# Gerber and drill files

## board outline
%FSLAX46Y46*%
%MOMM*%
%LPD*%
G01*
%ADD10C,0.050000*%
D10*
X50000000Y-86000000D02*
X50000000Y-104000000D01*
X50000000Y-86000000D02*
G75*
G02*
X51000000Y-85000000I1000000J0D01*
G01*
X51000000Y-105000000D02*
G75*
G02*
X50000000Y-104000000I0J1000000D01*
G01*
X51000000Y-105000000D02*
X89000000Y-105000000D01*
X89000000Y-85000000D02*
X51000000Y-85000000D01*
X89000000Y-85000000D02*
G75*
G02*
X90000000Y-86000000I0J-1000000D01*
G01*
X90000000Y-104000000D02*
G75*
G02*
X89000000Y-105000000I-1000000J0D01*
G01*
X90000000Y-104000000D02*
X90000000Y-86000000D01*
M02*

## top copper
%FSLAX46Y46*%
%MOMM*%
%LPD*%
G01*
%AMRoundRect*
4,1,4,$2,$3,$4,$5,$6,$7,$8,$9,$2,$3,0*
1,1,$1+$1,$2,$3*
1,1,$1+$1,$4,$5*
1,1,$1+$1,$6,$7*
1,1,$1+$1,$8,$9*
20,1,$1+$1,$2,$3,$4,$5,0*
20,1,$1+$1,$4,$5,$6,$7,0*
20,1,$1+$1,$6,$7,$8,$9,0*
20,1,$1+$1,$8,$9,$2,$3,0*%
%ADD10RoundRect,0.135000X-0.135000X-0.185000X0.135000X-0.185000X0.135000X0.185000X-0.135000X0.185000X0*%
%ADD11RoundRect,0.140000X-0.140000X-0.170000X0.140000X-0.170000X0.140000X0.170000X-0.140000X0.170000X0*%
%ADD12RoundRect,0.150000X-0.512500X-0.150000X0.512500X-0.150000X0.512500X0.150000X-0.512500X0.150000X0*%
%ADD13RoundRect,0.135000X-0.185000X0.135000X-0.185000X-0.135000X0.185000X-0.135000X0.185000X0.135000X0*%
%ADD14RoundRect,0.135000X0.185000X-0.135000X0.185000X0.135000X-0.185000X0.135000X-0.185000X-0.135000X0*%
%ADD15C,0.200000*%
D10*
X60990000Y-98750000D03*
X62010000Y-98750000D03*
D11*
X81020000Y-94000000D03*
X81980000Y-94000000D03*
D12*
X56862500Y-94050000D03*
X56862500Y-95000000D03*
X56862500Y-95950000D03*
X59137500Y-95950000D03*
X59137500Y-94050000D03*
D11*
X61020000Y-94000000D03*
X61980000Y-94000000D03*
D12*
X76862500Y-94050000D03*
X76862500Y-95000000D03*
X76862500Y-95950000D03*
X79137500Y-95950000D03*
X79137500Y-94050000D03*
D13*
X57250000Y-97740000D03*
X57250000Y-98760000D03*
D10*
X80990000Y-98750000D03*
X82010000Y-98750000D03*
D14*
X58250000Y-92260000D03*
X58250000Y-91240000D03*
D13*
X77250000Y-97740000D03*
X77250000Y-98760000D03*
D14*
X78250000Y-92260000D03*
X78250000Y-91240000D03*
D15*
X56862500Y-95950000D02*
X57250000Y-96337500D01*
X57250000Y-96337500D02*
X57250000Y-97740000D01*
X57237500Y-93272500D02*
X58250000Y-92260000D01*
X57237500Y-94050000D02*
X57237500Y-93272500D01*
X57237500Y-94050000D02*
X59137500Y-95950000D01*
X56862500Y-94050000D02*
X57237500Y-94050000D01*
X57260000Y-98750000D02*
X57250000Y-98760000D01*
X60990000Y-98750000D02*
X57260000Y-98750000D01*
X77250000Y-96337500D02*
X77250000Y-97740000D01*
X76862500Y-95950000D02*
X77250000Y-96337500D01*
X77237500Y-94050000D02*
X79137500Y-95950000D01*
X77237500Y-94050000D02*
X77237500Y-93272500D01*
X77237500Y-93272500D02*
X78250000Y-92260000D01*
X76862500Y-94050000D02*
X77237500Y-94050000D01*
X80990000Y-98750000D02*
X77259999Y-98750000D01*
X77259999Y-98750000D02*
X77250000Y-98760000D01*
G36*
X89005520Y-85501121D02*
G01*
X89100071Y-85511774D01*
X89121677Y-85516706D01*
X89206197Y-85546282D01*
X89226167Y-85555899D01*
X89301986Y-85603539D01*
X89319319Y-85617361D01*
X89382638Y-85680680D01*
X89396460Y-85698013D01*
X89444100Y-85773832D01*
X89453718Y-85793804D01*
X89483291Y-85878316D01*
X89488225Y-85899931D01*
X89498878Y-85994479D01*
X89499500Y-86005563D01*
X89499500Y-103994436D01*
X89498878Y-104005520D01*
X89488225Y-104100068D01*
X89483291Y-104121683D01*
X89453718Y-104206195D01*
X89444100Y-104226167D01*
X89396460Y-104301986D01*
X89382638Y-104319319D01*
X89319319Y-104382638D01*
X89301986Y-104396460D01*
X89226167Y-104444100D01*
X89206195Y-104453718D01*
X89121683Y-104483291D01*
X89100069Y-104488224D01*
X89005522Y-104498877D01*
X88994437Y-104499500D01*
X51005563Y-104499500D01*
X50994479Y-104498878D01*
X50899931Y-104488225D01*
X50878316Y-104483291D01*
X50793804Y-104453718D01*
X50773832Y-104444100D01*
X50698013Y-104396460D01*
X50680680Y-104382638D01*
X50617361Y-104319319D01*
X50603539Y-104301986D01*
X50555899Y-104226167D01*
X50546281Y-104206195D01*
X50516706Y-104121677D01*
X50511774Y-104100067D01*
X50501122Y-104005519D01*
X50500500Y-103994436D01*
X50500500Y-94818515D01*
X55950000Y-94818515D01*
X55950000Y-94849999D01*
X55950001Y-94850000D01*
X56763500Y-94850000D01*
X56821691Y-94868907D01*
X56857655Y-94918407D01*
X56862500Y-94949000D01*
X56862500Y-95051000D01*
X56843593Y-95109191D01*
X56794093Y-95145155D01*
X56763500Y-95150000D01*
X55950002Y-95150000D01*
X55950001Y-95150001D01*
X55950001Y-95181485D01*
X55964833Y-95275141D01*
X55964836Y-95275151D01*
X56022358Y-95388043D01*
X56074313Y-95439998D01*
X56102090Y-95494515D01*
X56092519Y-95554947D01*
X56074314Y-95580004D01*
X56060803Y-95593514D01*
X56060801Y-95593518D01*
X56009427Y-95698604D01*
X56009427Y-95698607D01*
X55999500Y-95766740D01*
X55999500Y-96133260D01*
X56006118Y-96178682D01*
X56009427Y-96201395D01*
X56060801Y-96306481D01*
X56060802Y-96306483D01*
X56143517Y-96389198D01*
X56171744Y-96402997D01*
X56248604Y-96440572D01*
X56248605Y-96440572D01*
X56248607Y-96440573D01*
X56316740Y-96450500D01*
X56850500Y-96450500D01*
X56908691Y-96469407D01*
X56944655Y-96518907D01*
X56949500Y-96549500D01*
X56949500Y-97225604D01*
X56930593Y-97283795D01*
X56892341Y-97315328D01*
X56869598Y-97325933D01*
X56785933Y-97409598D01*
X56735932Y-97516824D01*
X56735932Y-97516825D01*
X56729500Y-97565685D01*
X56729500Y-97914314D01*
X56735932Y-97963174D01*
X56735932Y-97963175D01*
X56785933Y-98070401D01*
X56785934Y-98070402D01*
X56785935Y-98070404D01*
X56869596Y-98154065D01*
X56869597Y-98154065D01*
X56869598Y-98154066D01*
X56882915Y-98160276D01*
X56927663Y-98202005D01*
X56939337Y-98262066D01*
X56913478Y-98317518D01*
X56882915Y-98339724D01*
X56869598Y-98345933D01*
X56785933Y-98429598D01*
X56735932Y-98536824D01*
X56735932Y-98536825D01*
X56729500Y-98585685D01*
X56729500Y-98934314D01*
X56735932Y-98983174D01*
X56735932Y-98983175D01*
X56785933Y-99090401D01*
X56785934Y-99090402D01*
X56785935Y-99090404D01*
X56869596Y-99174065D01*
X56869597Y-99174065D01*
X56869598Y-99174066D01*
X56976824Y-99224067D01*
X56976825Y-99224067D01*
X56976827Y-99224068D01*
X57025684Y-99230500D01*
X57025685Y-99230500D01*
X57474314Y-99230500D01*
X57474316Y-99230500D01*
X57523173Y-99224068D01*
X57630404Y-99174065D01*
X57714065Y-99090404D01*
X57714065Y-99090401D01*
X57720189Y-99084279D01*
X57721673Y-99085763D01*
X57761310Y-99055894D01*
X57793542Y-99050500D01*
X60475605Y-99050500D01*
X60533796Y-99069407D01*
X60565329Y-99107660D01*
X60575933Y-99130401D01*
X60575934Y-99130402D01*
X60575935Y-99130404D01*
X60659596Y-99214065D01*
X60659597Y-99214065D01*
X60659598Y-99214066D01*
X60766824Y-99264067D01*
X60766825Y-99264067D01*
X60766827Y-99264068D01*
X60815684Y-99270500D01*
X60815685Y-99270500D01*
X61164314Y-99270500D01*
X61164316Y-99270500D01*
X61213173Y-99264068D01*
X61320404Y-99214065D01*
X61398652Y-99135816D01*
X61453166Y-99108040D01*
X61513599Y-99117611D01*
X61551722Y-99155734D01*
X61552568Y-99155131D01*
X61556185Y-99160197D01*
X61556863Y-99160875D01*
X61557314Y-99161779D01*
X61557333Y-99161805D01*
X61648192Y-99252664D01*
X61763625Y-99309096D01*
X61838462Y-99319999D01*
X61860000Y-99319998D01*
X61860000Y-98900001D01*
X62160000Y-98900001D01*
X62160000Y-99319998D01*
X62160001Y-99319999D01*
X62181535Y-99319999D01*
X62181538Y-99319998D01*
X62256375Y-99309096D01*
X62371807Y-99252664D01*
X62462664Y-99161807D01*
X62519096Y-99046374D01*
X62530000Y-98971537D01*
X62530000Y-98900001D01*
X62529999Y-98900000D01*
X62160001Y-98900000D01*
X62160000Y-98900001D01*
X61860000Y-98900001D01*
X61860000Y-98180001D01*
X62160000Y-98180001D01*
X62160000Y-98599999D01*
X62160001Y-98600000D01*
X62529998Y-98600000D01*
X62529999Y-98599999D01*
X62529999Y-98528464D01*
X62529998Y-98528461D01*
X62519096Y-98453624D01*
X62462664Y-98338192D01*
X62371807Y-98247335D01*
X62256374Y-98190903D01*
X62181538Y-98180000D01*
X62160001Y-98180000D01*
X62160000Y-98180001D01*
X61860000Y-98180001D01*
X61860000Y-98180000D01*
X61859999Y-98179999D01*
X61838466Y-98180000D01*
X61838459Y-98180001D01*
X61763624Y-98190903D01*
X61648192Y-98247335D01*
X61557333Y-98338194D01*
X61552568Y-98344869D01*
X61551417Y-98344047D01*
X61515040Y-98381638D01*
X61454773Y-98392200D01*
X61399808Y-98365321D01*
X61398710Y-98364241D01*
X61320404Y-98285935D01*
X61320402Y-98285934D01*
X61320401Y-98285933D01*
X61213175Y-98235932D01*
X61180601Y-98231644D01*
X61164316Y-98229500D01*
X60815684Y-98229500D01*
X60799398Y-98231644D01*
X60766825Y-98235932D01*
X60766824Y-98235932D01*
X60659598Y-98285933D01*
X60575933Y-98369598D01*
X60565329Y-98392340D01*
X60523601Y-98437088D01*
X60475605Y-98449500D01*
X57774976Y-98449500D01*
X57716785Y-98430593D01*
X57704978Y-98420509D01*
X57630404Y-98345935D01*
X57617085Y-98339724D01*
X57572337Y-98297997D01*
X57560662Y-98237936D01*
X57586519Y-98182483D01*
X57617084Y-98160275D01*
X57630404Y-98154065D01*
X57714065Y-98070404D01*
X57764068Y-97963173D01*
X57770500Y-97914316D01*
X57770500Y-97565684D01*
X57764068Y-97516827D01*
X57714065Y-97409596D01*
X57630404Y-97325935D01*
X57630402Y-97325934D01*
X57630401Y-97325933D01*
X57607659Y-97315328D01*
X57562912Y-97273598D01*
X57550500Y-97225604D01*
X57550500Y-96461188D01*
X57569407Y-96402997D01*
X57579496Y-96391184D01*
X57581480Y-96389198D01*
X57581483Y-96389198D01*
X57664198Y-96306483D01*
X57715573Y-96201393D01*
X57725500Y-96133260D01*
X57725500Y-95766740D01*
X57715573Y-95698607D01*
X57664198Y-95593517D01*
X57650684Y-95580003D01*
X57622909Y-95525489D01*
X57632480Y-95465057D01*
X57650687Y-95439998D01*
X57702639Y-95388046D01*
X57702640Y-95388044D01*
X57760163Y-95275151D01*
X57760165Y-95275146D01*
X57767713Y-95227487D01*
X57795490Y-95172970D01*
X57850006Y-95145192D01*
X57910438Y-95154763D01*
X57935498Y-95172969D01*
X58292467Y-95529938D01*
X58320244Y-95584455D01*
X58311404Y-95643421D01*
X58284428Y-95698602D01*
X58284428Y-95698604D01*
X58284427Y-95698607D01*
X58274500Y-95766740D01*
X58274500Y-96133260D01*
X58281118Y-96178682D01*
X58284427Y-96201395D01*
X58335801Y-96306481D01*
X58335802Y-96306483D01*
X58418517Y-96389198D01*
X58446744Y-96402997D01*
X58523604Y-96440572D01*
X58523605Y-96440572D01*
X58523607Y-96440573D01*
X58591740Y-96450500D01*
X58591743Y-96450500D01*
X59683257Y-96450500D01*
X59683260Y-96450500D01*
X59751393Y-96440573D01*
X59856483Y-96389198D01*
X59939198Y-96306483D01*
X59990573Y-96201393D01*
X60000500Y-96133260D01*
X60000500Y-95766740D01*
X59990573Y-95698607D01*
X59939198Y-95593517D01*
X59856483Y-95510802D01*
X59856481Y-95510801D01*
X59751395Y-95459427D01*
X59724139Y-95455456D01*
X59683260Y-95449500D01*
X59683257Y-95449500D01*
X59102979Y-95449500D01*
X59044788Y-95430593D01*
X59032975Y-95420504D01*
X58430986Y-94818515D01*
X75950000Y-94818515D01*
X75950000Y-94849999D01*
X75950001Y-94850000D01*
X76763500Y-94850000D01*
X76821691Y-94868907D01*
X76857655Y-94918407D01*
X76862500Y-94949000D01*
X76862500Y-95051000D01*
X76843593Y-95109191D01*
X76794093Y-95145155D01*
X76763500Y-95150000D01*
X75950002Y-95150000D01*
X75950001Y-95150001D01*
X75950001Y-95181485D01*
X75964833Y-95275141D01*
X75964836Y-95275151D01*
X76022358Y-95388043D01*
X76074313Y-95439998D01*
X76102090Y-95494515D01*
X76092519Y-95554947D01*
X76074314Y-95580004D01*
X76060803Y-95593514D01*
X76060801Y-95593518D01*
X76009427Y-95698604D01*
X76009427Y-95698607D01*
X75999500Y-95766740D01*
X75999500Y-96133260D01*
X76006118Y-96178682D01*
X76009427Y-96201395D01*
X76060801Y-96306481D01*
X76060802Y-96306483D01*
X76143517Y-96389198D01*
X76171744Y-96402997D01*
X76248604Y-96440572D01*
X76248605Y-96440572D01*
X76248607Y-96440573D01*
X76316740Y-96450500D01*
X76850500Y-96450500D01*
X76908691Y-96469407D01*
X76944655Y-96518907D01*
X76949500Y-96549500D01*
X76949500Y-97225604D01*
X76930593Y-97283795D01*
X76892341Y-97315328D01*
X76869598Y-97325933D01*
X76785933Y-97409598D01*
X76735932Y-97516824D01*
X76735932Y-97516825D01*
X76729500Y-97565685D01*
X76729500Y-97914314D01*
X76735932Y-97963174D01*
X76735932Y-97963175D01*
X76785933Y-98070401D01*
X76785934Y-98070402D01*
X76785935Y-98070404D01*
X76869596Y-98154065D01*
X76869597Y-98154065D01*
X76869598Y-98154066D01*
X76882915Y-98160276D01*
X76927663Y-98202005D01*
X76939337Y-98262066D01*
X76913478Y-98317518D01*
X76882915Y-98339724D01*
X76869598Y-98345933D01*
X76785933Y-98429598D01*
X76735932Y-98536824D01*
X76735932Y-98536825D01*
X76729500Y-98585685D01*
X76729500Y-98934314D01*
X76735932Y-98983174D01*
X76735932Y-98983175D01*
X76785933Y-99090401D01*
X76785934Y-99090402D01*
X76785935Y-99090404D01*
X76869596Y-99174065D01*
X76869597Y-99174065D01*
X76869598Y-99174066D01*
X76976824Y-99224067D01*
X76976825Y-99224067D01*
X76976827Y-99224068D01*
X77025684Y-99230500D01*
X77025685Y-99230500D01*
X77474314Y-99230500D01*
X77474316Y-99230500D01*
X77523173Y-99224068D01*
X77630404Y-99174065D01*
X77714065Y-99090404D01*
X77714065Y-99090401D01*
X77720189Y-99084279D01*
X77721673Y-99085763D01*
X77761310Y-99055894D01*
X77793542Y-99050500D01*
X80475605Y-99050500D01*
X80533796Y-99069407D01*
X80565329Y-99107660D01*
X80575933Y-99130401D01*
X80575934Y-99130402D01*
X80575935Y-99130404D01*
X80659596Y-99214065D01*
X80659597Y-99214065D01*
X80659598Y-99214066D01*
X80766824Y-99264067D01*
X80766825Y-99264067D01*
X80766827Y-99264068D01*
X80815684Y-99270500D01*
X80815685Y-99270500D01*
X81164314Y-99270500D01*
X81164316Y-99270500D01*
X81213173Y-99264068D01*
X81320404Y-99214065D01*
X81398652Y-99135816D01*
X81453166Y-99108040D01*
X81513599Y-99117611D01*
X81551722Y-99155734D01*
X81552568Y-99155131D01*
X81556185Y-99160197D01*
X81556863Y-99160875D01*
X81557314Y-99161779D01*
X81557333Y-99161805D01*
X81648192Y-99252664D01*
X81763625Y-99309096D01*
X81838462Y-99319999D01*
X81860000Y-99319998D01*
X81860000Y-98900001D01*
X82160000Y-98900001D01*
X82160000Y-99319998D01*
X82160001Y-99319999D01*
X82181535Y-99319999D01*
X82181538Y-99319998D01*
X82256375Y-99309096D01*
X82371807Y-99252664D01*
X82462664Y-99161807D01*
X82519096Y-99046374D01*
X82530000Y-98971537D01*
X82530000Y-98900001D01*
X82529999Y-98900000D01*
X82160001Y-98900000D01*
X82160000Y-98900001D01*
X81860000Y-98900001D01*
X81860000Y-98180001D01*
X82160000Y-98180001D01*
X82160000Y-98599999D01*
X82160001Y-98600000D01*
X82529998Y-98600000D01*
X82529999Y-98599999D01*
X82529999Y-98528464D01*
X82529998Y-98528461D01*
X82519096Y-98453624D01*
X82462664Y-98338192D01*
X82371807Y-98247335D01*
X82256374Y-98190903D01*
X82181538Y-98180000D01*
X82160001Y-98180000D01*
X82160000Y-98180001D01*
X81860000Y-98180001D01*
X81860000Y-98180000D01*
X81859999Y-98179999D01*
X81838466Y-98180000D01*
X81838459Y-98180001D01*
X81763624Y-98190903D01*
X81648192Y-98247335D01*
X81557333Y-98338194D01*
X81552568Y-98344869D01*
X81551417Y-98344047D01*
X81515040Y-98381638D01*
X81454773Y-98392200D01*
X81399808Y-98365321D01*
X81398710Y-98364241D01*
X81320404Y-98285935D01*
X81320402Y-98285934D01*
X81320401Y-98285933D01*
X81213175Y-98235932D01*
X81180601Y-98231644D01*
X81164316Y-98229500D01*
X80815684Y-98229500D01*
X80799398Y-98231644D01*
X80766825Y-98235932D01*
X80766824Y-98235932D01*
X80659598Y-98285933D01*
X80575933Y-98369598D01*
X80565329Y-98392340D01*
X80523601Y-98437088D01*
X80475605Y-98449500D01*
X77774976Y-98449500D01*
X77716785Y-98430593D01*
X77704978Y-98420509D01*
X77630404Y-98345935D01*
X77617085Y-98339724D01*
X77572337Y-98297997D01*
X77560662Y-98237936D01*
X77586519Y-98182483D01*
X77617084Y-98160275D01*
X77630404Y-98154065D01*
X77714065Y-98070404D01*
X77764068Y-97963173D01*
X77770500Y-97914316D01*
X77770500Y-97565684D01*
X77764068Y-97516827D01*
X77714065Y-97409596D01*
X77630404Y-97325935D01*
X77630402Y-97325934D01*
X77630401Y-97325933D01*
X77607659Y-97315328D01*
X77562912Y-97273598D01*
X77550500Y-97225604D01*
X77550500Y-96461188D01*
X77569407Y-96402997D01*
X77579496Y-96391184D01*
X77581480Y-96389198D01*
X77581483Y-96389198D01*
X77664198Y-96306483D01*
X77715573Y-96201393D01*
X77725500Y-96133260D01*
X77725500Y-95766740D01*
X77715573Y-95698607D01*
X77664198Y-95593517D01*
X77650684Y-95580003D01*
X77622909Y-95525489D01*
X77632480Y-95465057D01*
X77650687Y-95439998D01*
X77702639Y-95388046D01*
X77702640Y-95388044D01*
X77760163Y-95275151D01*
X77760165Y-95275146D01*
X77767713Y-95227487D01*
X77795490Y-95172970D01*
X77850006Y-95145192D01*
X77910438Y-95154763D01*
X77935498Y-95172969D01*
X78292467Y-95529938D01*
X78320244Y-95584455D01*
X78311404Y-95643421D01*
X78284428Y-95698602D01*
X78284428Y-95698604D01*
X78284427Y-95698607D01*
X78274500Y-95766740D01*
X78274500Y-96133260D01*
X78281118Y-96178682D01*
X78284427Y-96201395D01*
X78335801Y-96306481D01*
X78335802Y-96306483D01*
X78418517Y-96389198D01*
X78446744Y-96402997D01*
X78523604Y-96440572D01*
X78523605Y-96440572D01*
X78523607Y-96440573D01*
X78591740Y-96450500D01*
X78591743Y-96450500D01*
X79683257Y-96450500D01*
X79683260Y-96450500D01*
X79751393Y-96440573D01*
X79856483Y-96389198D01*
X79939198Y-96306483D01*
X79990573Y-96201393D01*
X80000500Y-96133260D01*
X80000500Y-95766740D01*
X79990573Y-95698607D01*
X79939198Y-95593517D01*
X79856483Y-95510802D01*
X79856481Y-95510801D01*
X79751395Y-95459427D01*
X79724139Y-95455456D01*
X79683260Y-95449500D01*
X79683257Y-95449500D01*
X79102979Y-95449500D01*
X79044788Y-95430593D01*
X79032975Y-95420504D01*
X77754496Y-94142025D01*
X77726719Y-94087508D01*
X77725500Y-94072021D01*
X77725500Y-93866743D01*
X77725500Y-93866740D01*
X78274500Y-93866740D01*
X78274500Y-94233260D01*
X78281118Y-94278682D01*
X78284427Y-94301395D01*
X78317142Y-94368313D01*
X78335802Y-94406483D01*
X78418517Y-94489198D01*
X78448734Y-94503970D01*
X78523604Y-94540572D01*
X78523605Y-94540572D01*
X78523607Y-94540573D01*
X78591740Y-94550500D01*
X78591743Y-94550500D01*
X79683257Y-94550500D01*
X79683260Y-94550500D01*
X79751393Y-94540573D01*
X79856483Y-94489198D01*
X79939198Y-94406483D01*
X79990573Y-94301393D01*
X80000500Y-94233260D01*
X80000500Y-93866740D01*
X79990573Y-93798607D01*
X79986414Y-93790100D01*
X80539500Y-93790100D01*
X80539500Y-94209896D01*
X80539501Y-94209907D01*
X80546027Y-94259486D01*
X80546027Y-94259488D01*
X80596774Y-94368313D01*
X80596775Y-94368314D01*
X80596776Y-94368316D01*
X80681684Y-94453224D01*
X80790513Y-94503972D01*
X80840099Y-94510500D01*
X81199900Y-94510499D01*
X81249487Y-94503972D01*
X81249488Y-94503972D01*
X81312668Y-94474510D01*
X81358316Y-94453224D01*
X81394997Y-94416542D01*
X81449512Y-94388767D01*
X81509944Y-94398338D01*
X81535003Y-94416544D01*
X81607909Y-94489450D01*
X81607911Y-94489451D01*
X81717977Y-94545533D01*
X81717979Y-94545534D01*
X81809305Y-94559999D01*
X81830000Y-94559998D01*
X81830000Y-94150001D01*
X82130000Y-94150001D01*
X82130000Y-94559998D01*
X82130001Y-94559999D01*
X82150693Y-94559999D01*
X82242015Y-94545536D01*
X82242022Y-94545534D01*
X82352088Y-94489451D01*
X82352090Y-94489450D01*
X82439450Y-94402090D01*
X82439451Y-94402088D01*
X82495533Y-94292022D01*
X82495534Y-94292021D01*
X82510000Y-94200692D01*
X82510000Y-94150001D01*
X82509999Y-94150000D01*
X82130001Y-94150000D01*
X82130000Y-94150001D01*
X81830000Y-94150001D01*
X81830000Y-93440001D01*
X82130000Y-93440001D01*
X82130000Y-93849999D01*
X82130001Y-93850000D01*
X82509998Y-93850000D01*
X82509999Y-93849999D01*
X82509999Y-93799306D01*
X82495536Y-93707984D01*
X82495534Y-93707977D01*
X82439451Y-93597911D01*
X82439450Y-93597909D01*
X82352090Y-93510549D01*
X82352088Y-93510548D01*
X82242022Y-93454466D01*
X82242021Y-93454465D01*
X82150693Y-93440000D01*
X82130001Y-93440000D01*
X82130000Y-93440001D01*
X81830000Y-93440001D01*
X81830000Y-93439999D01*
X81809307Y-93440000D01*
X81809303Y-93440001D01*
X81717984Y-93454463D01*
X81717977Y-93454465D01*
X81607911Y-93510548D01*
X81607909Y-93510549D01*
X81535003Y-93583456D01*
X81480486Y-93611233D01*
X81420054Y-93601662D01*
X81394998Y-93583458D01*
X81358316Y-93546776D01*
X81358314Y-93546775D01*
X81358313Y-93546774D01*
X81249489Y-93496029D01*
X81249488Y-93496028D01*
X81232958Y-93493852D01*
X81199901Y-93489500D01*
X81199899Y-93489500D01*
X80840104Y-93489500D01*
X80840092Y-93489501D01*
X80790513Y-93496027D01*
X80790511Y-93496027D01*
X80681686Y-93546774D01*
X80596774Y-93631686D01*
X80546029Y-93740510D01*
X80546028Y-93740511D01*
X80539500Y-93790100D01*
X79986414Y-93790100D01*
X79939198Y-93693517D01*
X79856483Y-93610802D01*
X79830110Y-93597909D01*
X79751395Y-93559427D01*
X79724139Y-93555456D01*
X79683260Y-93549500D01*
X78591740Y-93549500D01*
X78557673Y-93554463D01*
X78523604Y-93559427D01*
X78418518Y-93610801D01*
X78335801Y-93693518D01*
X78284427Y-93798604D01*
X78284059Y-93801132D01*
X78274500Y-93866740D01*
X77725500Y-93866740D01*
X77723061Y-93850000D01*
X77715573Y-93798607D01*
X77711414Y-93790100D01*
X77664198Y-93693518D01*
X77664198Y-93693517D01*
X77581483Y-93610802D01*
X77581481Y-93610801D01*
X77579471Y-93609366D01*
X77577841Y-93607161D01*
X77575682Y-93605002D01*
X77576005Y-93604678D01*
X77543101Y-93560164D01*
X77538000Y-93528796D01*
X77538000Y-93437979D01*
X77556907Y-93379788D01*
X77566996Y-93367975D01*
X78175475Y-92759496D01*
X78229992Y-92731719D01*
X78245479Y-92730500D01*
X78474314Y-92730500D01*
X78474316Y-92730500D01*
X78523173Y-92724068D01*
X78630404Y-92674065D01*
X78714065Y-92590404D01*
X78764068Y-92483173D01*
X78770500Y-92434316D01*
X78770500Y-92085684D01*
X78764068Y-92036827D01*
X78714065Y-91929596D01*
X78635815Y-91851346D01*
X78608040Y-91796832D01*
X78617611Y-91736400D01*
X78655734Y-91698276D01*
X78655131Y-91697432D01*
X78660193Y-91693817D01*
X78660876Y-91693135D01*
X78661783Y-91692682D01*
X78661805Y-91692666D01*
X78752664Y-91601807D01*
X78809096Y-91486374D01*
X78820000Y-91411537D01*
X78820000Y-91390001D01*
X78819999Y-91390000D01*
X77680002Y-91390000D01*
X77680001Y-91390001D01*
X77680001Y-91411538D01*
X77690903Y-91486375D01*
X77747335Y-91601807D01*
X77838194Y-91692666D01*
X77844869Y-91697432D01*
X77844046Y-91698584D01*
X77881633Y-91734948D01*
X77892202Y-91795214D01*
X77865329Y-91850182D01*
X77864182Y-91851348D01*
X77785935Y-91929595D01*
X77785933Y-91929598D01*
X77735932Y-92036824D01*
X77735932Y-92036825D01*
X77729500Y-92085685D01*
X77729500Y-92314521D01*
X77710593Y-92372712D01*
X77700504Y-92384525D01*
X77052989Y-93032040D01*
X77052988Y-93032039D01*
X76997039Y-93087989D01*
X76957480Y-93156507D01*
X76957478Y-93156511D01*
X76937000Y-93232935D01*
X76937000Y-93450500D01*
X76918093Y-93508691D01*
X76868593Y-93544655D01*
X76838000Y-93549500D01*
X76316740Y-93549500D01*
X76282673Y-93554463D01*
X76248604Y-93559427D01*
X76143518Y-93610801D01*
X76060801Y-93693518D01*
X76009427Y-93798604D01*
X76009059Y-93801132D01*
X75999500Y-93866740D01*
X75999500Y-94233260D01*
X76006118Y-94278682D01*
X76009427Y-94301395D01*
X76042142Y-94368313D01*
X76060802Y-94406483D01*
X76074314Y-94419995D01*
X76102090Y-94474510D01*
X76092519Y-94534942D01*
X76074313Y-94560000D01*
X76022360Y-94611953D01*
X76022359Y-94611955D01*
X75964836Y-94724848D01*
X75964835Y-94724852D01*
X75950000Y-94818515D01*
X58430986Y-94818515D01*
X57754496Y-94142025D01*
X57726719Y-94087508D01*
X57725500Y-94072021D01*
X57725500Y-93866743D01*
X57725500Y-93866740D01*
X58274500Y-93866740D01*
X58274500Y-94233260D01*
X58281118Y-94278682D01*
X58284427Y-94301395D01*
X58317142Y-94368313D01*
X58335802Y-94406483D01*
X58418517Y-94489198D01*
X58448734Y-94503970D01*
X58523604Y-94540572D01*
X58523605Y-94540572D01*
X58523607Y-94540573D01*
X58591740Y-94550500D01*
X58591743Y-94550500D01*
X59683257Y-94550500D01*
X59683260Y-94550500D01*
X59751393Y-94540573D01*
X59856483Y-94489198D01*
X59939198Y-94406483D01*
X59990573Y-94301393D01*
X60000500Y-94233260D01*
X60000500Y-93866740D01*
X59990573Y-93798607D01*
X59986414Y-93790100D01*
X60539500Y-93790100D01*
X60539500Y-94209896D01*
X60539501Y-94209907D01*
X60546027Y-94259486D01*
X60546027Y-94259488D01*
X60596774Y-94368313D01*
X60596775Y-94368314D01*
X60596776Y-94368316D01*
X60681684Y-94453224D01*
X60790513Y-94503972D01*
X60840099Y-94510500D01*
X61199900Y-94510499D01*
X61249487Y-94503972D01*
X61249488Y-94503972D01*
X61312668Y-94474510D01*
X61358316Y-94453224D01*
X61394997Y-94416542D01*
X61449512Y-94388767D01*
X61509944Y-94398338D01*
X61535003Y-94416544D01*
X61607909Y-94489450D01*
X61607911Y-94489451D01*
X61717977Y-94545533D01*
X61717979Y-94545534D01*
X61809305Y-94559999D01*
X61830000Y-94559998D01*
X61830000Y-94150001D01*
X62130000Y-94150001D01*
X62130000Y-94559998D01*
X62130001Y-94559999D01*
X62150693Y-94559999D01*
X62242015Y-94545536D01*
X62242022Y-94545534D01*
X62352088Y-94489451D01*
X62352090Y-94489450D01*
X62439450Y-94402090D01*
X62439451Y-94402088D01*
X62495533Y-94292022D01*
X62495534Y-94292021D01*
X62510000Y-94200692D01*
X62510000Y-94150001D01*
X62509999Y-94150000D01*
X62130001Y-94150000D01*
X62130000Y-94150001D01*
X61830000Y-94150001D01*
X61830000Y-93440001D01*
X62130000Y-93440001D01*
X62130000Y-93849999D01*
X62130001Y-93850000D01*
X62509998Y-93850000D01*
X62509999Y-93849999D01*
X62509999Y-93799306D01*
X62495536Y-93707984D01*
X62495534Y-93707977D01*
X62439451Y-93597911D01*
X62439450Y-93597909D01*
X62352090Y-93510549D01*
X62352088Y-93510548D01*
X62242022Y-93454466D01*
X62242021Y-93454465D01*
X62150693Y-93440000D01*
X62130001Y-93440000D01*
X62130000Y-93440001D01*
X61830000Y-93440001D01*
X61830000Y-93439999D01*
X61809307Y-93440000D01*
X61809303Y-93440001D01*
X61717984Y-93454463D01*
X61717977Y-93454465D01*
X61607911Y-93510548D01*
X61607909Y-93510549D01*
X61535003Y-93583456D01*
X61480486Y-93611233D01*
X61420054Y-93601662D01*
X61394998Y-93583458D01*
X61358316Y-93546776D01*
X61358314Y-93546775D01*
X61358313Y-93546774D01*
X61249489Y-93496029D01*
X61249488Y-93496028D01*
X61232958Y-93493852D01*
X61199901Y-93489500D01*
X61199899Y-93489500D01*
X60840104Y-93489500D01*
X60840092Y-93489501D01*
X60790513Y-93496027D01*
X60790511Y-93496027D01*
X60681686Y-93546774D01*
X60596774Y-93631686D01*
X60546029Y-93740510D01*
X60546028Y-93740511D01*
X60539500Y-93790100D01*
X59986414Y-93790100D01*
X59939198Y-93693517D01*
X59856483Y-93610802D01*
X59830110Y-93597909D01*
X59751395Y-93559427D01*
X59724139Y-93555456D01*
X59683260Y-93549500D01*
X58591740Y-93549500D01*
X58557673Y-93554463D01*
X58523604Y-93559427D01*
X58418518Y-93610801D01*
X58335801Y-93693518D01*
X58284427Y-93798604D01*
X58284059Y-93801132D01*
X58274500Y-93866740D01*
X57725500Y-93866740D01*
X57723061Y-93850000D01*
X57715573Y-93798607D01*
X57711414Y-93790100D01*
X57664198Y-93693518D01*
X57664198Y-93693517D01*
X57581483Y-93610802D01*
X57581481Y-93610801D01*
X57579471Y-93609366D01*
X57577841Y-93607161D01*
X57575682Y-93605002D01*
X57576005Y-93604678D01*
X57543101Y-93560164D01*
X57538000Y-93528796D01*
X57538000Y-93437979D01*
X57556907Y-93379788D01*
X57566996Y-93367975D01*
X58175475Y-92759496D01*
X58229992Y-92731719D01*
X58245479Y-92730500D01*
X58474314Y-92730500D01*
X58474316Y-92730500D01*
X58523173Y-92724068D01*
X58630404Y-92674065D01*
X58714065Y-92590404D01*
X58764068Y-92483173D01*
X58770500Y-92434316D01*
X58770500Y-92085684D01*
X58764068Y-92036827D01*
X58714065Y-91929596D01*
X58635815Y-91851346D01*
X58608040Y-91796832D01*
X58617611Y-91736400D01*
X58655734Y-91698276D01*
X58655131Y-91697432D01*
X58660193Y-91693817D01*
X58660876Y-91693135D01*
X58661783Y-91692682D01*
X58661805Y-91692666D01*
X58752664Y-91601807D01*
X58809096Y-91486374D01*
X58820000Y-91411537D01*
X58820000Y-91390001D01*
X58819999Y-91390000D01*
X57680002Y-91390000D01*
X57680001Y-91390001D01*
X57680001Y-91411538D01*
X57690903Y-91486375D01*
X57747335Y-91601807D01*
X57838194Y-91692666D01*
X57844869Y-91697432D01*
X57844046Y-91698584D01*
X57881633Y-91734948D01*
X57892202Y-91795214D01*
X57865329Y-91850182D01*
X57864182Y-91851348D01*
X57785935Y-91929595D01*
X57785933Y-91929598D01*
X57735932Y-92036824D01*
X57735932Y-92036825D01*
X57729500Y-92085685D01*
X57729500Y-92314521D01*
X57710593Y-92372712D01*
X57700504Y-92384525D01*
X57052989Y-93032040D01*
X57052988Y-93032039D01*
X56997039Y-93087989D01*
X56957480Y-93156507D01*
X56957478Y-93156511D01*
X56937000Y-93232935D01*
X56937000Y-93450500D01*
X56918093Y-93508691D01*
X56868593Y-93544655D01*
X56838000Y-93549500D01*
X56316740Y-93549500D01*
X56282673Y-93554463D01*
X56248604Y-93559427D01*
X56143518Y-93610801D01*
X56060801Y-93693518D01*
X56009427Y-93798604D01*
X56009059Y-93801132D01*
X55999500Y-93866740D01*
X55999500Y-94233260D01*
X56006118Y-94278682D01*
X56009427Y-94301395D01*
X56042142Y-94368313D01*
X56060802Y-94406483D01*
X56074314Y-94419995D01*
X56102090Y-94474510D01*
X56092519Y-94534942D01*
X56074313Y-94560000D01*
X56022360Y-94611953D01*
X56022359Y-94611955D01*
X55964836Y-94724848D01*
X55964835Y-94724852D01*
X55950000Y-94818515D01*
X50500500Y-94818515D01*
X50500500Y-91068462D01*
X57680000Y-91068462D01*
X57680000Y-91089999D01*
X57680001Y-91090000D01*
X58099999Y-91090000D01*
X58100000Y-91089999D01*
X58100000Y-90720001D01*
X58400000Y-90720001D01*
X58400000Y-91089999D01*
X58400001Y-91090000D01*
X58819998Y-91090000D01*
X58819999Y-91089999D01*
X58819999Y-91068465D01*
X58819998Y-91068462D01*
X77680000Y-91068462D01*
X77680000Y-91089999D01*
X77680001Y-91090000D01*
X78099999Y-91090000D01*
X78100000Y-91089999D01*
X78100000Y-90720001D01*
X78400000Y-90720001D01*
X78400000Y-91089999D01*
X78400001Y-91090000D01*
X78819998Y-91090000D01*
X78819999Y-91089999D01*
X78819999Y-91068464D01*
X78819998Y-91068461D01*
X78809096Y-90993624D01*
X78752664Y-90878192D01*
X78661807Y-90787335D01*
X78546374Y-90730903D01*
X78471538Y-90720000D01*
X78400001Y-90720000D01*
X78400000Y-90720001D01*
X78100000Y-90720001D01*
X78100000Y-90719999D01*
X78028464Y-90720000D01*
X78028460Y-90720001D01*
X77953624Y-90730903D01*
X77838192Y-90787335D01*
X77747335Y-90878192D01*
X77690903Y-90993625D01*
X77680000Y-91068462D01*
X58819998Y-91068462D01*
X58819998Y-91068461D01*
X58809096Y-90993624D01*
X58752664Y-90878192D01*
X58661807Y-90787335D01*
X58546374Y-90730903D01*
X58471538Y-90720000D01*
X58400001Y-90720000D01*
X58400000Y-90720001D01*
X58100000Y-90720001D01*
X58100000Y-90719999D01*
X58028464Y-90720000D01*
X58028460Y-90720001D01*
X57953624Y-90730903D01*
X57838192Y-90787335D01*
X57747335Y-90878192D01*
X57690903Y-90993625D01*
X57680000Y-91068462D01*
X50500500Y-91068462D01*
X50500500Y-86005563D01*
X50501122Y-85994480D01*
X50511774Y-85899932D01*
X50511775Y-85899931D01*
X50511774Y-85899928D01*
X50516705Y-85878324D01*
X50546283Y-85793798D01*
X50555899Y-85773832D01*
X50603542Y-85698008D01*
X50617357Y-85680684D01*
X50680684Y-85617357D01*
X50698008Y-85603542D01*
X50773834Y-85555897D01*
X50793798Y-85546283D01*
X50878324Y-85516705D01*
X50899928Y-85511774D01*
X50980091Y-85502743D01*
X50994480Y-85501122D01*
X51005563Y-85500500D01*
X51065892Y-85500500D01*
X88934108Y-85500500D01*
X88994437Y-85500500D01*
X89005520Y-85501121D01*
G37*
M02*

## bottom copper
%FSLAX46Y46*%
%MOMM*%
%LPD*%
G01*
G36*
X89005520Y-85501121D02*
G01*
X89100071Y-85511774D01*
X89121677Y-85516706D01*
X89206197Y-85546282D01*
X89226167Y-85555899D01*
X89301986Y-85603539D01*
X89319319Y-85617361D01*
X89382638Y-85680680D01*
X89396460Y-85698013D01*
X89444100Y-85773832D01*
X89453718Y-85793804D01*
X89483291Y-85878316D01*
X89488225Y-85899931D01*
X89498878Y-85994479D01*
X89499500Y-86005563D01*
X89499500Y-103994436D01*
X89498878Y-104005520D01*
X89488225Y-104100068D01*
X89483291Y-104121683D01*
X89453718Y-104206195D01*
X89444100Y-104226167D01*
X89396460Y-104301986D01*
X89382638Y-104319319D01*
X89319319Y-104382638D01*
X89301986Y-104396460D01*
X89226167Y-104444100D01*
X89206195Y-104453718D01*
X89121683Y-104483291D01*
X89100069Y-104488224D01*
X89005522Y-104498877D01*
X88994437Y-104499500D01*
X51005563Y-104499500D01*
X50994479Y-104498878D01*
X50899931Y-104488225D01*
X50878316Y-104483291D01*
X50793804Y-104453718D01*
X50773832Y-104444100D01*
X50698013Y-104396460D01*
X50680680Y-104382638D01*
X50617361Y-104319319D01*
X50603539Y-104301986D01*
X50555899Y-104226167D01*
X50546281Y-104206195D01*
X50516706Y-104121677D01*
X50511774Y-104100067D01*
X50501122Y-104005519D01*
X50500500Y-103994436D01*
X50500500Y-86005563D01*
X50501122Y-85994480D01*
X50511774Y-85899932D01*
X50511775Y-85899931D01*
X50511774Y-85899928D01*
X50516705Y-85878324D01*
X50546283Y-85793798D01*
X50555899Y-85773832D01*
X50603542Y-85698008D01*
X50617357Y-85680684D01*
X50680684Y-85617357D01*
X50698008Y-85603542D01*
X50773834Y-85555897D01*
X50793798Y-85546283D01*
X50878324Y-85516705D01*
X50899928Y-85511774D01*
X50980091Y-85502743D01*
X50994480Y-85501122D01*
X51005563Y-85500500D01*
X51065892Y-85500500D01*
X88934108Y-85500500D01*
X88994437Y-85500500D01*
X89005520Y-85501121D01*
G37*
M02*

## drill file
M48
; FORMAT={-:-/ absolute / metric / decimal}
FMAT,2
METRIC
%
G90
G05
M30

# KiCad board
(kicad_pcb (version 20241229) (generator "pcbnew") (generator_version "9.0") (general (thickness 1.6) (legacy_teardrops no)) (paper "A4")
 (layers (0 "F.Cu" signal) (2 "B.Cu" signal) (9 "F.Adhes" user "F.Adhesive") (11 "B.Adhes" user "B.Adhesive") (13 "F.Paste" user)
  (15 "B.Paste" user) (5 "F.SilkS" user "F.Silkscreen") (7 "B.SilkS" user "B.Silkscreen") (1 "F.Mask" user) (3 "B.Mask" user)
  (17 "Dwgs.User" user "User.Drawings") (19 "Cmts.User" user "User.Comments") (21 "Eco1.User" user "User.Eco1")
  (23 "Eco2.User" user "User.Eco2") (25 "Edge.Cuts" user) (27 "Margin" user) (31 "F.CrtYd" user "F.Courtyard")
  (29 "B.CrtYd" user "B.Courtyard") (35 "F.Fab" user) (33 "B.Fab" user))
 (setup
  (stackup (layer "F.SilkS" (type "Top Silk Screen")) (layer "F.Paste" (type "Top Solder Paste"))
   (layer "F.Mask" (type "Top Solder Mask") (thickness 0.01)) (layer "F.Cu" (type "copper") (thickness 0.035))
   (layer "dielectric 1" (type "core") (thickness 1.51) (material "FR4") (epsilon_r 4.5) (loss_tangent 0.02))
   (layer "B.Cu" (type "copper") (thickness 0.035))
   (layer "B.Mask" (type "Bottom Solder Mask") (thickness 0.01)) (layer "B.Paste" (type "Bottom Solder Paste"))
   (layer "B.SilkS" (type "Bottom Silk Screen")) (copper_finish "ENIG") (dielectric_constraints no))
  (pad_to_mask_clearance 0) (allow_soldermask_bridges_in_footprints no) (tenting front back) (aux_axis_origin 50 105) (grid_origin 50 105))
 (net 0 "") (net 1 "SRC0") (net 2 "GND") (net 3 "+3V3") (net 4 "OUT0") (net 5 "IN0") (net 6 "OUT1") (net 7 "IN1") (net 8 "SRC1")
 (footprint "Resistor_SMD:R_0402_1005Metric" (layer "F.Cu") (at 61.5 98.75)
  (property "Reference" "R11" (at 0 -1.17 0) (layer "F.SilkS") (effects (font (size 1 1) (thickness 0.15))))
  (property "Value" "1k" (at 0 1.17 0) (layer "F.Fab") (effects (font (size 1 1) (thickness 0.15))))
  (pad "1" smd roundrect (at -0.51 0) (size 0.54 0.64) (layers "F.Cu" "F.Mask" "F.Paste") (roundrect_rratio 0.25) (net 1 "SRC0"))
  (pad "2" smd roundrect (at 0.51 0) (size 0.54 0.64) (layers "F.Cu" "F.Mask" "F.Paste") (roundrect_rratio 0.25) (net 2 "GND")))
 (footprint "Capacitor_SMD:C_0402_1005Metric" (layer "F.Cu") (at 81.5 94)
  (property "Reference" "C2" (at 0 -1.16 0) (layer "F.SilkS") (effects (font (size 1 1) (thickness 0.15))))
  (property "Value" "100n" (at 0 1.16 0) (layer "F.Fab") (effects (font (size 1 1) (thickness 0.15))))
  (pad "1" smd roundrect (at -0.48 0) (size 0.56 0.62) (layers "F.Cu" "F.Mask" "F.Paste") (roundrect_rratio 0.25) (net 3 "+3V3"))
  (pad "2" smd roundrect (at 0.48 0) (size 0.56 0.62) (layers "F.Cu" "F.Mask" "F.Paste") (roundrect_rratio 0.25) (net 2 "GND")))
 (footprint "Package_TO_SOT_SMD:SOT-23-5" (layer "F.Cu") (at 58 95)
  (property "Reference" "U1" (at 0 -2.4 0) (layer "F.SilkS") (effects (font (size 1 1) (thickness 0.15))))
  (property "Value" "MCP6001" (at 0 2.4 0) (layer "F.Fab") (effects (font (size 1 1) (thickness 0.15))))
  (pad "1" smd roundrect (at -1.1375 -0.95) (size 1.325 0.6) (layers "F.Cu" "F.Mask" "F.Paste") (roundrect_rratio 0.25) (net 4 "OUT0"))
  (pad "2" smd roundrect (at -1.1375 0) (size 1.325 0.6) (layers "F.Cu" "F.Mask" "F.Paste") (roundrect_rratio 0.25) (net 2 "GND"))
  (pad "3" smd roundrect (at -1.1375 0.95) (size 1.325 0.6) (layers "F.Cu" "F.Mask" "F.Paste") (roundrect_rratio 0.25) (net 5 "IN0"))
  (pad "4" smd roundrect (at 1.1375 0.95) (size 1.325 0.6) (layers "F.Cu" "F.Mask" "F.Paste") (roundrect_rratio 0.25) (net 4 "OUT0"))
  (pad "5" smd roundrect (at 1.1375 -0.95) (size 1.325 0.6) (layers "F.Cu" "F.Mask" "F.Paste") (roundrect_rratio 0.25) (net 3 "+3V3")))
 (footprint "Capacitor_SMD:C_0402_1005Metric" (layer "F.Cu") (at 61.5 94)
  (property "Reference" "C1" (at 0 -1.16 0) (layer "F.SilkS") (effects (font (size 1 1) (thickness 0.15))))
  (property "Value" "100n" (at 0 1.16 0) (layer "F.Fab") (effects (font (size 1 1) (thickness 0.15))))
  (pad "1" smd roundrect (at -0.48 0) (size 0.56 0.62) (layers "F.Cu" "F.Mask" "F.Paste") (roundrect_rratio 0.25) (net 3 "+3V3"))
  (pad "2" smd roundrect (at 0.48 0) (size 0.56 0.62) (layers "F.Cu" "F.Mask" "F.Paste") (roundrect_rratio 0.25) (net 2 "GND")))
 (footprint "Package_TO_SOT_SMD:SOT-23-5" (layer "F.Cu") (at 78 95)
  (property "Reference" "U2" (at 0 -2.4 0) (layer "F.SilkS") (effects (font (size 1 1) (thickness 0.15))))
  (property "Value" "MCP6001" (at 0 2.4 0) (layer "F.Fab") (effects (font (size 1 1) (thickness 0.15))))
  (pad "1" smd roundrect (at -1.1375 -0.95) (size 1.325 0.6) (layers "F.Cu" "F.Mask" "F.Paste") (roundrect_rratio 0.25) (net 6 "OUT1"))
  (pad "2" smd roundrect (at -1.1375 0) (size 1.325 0.6) (layers "F.Cu" "F.Mask" "F.Paste") (roundrect_rratio 0.25) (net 2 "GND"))
  (pad "3" smd roundrect (at -1.1375 0.95) (size 1.325 0.6) (layers "F.Cu" "F.Mask" "F.Paste") (roundrect_rratio 0.25) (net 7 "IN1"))
  (pad "4" smd roundrect (at 1.1375 0.95) (size 1.325 0.6) (layers "F.Cu" "F.Mask" "F.Paste") (roundrect_rratio 0.25) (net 6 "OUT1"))
  (pad "5" smd roundrect (at 1.1375 -0.95) (size 1.325 0.6) (layers "F.Cu" "F.Mask" "F.Paste") (roundrect_rratio 0.25) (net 3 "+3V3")))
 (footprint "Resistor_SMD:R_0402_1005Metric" (layer "F.Cu") (at 57.25 98.25 -90)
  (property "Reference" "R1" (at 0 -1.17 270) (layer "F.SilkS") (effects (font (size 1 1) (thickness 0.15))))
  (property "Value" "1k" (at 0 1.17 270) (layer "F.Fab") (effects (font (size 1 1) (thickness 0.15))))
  (pad "1" smd roundrect (at -0.51 0 270) (size 0.54 0.64) (layers "F.Cu" "F.Mask" "F.Paste") (roundrect_rratio 0.25) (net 5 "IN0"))
  (pad "2" smd roundrect (at 0.51 0 270) (size 0.54 0.64) (layers "F.Cu" "F.Mask" "F.Paste") (roundrect_rratio 0.25) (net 1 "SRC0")))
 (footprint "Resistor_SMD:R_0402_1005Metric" (layer "F.Cu") (at 81.5 98.75)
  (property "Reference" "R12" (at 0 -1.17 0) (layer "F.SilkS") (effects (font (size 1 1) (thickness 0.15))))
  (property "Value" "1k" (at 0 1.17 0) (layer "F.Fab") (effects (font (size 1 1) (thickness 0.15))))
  (pad "1" smd roundrect (at -0.51 0) (size 0.54 0.64) (layers "F.Cu" "F.Mask" "F.Paste") (roundrect_rratio 0.25) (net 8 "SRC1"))
  (pad "2" smd roundrect (at 0.51 0) (size 0.54 0.64) (layers "F.Cu" "F.Mask" "F.Paste") (roundrect_rratio 0.25) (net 2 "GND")))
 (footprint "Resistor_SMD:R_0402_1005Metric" (layer "F.Cu") (at 58.25 91.75 90)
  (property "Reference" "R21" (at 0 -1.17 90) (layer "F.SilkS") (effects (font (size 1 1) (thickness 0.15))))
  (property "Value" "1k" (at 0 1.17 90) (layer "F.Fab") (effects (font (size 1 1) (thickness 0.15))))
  (pad "1" smd roundrect (at -0.51 0 90) (size 0.54 0.64) (layers "F.Cu" "F.Mask" "F.Paste") (roundrect_rratio 0.25) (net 4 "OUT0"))
  (pad "2" smd roundrect (at 0.51 0 90) (size 0.54 0.64) (layers "F.Cu" "F.Mask" "F.Paste") (roundrect_rratio 0.25) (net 2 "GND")))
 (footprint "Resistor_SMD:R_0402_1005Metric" (layer "F.Cu") (at 77.25 98.25 -90)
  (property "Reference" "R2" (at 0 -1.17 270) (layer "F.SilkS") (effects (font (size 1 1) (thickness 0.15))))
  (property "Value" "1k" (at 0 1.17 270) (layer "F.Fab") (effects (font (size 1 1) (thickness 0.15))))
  (pad "1" smd roundrect (at -0.51 0 270) (size 0.54 0.64) (layers "F.Cu" "F.Mask" "F.Paste") (roundrect_rratio 0.25) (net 7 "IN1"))
  (pad "2" smd roundrect (at 0.51 0 270) (size 0.54 0.64) (layers "F.Cu" "F.Mask" "F.Paste") (roundrect_rratio 0.25) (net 8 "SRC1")))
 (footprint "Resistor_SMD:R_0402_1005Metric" (layer "F.Cu") (at 78.25 91.75 90)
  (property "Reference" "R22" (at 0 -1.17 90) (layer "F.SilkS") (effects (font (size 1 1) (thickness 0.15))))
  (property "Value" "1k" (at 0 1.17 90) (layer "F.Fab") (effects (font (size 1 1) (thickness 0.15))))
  (pad "1" smd roundrect (at -0.51 0 90) (size 0.54 0.64) (layers "F.Cu" "F.Mask" "F.Paste") (roundrect_rratio 0.25) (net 6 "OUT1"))
  (pad "2" smd roundrect (at 0.51 0 90) (size 0.54 0.64) (layers "F.Cu" "F.Mask" "F.Paste") (roundrect_rratio 0.25) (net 2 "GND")))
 (gr_line (start 50 86) (end 50 104) (stroke (width 0.05) (type default)) (layer "Edge.Cuts"))
 (gr_arc (start 50 86) (mid 50.292893 85.292893) (end 51 85) (stroke (width 0.05) (type default)) (layer "Edge.Cuts"))
 (gr_arc (start 51 105) (mid 50.292893 104.707107) (end 50 104) (stroke (width 0.05) (type default)) (layer "Edge.Cuts"))
 (gr_line (start 51 105) (end 89 105) (stroke (width 0.05) (type default)) (layer "Edge.Cuts"))
 (gr_line (start 89 85) (end 51 85) (stroke (width 0.05) (type default)) (layer "Edge.Cuts"))
 (gr_arc (start 89 85) (mid 89.707107 85.292893) (end 90 86) (stroke (width 0.05) (type default)) (layer "Edge.Cuts"))
 (gr_arc (start 90 104) (mid 89.707107 104.707107) (end 89 105) (stroke (width 0.05) (type default)) (layer "Edge.Cuts"))
 (gr_line (start 90 104) (end 90 86) (stroke (width 0.05) (type default)) (layer "Edge.Cuts"))
 (segment (start 56.8625 95.95) (end 57.25 96.3375) (width 0.2) (locked yes) (layer "F.Cu") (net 5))
 (segment (start 57.25 96.3375) (end 57.25 97.74) (width 0.2) (locked yes) (layer "F.Cu") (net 5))
 (segment (start 57.2375 93.2725) (end 58.25 92.26) (width 0.2) (locked yes) (layer "F.Cu") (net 4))
 (segment (start 57.2375 94.05) (end 57.2375 93.2725) (width 0.2) (locked yes) (layer "F.Cu") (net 4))
 (segment (start 57.2375 94.05) (end 59.1375 95.95) (width 0.2) (locked yes) (layer "F.Cu") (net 4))
 (segment (start 56.8625 94.05) (end 57.2375 94.05) (width 0.2) (locked yes) (layer "F.Cu") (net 4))
 (segment (start 57.26 98.75) (end 57.25 98.76) (width 0.2) (locked yes) (layer "F.Cu") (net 1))
 (segment (start 60.99 98.75) (end 57.26 98.75) (width 0.2) (locked yes) (layer "F.Cu") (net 1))
 (segment (start 77.25 96.3375) (end 77.25 97.74) (width 0.2) (locked yes) (layer "F.Cu") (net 7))
 (segment (start 76.8625 95.95) (end 77.25 96.3375) (width 0.2) (locked yes) (layer "F.Cu") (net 7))
 (segment (start 77.2375 94.05) (end 79.1375 95.95) (width 0.2) (locked yes) (layer "F.Cu") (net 6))
 (segment (start 77.2375 94.05) (end 77.2375 93.2725) (width 0.2) (locked yes) (layer "F.Cu") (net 6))
 (segment (start 77.2375 93.2725) (end 78.25 92.26) (width 0.2) (locked yes) (layer "F.Cu") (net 6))
 (segment (start 76.8625 94.05) (end 77.2375 94.05) (width 0.2) (locked yes) (layer "F.Cu") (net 6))
 (segment (start 80.99 98.75) (end 77.259999 98.75) (width 0.2) (locked yes) (layer "F.Cu") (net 8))
 (segment (start 77.259999 98.75) (end 77.25 98.76) (width 0.2) (locked yes) (layer "F.Cu") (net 8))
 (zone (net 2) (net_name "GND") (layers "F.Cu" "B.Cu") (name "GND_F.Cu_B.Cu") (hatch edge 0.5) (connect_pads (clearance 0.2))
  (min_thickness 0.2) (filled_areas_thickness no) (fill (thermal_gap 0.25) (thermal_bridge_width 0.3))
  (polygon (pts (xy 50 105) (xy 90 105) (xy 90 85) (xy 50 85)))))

